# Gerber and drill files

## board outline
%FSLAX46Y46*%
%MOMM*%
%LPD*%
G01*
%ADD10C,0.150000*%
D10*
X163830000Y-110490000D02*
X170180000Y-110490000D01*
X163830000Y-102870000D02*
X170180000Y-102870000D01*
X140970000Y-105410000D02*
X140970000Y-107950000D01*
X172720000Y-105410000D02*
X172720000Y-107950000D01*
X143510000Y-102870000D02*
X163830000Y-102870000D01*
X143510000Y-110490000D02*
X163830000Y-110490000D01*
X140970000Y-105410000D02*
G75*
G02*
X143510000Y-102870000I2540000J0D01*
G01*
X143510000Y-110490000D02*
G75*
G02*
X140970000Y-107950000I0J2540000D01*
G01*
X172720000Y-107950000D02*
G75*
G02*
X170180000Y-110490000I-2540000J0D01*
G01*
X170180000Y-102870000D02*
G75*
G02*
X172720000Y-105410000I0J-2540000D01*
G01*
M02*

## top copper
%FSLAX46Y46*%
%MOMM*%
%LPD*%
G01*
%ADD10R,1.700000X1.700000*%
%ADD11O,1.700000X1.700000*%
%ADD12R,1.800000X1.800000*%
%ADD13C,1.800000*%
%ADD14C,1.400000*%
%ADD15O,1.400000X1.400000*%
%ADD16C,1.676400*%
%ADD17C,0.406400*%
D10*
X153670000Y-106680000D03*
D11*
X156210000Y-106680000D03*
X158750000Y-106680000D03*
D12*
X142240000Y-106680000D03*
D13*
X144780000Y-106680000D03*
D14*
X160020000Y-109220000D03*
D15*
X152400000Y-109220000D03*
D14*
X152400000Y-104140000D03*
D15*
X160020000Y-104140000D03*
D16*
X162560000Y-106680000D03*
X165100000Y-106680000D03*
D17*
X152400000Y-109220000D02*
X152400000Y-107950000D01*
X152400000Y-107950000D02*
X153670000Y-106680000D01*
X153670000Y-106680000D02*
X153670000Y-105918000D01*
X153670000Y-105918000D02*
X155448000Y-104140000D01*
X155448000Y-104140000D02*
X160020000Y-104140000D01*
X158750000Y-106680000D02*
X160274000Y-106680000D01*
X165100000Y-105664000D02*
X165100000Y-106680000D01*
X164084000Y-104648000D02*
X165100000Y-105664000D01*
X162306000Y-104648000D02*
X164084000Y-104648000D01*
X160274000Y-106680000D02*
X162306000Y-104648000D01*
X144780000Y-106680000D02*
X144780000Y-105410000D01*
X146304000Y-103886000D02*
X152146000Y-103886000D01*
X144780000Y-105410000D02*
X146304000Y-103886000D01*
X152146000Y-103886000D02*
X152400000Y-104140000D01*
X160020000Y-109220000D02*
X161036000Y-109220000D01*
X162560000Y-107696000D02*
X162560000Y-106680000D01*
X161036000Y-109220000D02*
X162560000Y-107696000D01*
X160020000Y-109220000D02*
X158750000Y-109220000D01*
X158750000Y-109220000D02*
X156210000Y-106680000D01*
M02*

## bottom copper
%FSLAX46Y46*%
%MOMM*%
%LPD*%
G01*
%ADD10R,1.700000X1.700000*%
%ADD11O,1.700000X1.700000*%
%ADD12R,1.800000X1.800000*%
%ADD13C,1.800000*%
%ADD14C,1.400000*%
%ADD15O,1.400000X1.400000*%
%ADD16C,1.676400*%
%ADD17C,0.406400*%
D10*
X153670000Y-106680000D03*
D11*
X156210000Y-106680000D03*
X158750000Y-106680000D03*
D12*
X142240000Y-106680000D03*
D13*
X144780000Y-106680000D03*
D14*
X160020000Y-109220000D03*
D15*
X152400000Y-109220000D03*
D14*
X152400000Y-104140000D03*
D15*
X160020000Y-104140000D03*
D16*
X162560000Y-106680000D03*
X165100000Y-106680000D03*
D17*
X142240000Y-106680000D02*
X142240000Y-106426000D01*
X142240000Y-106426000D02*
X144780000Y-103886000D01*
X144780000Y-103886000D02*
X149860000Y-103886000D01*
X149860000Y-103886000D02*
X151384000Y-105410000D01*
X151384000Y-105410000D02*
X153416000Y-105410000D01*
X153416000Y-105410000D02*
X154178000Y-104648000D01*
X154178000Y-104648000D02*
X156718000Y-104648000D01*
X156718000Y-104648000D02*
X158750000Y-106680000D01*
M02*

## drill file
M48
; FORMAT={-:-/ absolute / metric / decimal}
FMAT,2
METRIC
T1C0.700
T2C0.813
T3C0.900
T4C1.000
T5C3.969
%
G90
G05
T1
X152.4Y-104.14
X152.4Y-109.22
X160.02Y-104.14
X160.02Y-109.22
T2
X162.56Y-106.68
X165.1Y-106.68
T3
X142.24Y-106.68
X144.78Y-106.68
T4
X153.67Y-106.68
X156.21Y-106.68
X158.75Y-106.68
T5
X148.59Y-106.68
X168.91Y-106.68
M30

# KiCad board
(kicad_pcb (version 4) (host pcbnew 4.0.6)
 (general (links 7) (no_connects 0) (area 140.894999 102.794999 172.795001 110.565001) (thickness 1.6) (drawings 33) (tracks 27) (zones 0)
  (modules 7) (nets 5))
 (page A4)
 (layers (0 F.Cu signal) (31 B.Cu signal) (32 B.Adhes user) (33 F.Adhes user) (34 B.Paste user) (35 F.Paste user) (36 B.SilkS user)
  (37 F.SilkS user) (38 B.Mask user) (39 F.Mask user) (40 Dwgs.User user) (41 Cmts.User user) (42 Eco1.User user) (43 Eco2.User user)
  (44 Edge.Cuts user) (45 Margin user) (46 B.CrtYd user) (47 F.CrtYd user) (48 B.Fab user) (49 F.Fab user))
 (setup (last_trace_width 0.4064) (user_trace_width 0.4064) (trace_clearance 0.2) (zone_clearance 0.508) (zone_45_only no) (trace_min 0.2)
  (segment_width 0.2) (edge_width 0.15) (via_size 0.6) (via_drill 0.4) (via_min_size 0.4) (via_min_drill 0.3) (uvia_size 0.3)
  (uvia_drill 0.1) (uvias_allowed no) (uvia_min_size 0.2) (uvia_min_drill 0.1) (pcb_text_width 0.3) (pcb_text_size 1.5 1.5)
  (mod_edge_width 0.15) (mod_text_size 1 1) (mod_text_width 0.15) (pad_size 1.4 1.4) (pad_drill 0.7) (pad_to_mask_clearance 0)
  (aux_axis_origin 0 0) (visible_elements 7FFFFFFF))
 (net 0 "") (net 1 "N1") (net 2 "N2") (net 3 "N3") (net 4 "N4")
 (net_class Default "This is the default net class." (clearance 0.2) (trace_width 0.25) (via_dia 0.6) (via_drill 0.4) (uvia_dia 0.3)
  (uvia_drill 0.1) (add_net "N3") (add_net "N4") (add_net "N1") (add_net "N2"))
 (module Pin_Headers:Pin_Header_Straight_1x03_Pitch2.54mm (layer F.Cu) (at 153.67 106.68 90)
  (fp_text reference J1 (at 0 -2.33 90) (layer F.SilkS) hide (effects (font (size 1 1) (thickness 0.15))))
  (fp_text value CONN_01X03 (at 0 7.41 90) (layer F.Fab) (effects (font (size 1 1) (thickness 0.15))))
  (pad 1 thru_hole rect (at 0 0 90) (size 1.7 1.7) (drill 1) (layers *.Cu *.Mask) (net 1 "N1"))
  (pad 2 thru_hole oval (at 0 2.54 90) (size 1.7 1.7) (drill 1) (layers *.Cu *.Mask) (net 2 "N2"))
  (pad 3 thru_hole oval (at 0 5.08 90) (size 1.7 1.7) (drill 1) (layers *.Cu *.Mask) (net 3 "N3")))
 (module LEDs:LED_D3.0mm (layer F.Cu) (at 142.24 106.68)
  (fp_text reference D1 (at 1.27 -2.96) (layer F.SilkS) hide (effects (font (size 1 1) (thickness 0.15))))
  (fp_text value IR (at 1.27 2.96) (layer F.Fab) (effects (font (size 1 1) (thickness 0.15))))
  (pad 1 thru_hole rect (at 0 0) (size 1.8 1.8) (drill 0.9) (layers *.Cu B.Mask) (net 3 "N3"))
  (pad 2 thru_hole circle (at 2.54 0) (size 1.8 1.8) (drill 0.9) (layers *.Cu B.Mask) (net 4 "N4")))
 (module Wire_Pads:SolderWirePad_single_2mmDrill (layer F.Cu) (at 168.91 106.68)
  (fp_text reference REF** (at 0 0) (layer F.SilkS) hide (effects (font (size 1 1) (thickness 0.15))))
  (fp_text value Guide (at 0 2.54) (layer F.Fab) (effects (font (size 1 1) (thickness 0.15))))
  (pad "" np_thru_hole circle (at 0 0) (size 3.96875 3.96875) (drill 3.96875) (layers *.Cu *.Mask)))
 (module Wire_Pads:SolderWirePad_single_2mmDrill (layer F.Cu) (at 148.59 106.68)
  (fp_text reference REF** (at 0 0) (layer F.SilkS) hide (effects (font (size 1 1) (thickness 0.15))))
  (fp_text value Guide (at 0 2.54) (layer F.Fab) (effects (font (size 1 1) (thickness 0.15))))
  (pad "" np_thru_hole circle (at 0 0) (size 3.96875 3.96875) (drill 3.96875) (layers *.Cu *.Mask)))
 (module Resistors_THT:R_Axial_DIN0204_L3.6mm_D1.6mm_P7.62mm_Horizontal (layer F.Cu) (at 160.02 109.22 180)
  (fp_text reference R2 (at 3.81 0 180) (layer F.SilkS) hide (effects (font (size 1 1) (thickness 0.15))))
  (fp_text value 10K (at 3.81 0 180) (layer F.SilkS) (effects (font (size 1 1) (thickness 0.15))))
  (pad 1 thru_hole circle (at 0 0 180) (size 1.4 1.4) (drill 0.7) (layers *.Cu *.Mask) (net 2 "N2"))
  (pad 2 thru_hole oval (at 7.62 0 180) (size 1.4 1.4) (drill 0.7) (layers *.Cu *.Mask) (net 1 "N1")))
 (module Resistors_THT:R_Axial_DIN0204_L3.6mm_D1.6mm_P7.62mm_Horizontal (layer F.Cu) (at 152.4 104.14)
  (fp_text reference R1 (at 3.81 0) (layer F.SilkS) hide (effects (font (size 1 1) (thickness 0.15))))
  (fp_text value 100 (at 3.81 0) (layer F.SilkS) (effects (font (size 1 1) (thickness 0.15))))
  (pad 1 thru_hole circle (at 0 0) (size 1.4 1.4) (drill 0.7) (layers *.Cu *.Mask) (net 4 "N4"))
  (pad 2 thru_hole oval (at 7.62 0) (size 1.4 1.4) (drill 0.7) (layers *.Cu *.Mask) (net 1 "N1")))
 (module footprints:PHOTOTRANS (layer F.Cu) (at 163.83 106.68)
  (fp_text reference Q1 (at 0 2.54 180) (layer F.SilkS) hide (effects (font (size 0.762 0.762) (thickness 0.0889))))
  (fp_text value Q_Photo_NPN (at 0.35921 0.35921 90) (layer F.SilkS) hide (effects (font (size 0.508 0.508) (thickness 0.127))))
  (pad 1 thru_hole circle (at -1.27 0) (size 1.6764 1.6764) (drill 0.8128) (layers *.Cu B.Mask) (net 2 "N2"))
  (pad 2 thru_hole circle (at 1.27 0 45) (size 1.6764 1.6764) (drill 0.8128) (layers *.Cu B.Mask) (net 3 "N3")))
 (gr_line (start 163.83 110.49) (end 170.18 110.49) (angle 90) (layer Edge.Cuts) (width 0.15))
 (gr_line (start 163.83 102.87) (end 170.18 102.87) (angle 90) (layer Edge.Cuts) (width 0.15))
 (gr_line (start 140.97 105.41) (end 140.97 107.95) (angle 90) (layer Edge.Cuts) (width 0.15))
 (gr_line (start 172.72 105.41) (end 172.72 107.95) (angle 90) (layer Edge.Cuts) (width 0.15))
 (gr_line (start 143.51 102.87) (end 163.83 102.87) (angle 90) (layer Edge.Cuts) (width 0.15))
 (gr_line (start 143.51 110.49) (end 163.83 110.49) (angle 90) (layer Edge.Cuts) (width 0.15))
 (gr_arc (start 143.51 105.41) (end 140.97 105.41) (angle 90) (layer Edge.Cuts) (width 0.15))
 (gr_arc (start 143.51 107.95) (end 143.51 110.49) (angle 90) (layer Edge.Cuts) (width 0.15))
 (gr_arc (start 170.18 107.95) (end 172.72 107.95) (angle 90) (layer Edge.Cuts) (width 0.15))
 (gr_arc (start 170.18 105.41) (end 170.18 102.87) (angle 90) (layer Edge.Cuts) (width 0.15))
 (segment (start 152.4 109.22) (end 152.4 107.95) (width 0.4064) (layer F.Cu) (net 1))
 (segment (start 152.4 107.95) (end 153.67 106.68) (width 0.4064) (layer F.Cu) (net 1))
 (segment (start 153.67 106.68) (end 153.67 105.918) (width 0.4064) (layer F.Cu) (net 1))
 (segment (start 153.67 105.918) (end 155.448 104.14) (width 0.4064) (layer F.Cu) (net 1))
 (segment (start 155.448 104.14) (end 160.02 104.14) (width 0.4064) (layer F.Cu) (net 1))
 (segment (start 142.24 106.68) (end 142.24 106.426) (width 0.4064) (layer B.Cu) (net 3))
 (segment (start 142.24 106.426) (end 144.78 103.886) (width 0.4064) (layer B.Cu) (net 3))
 (segment (start 144.78 103.886) (end 149.86 103.886) (width 0.4064) (layer B.Cu) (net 3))
 (segment (start 149.86 103.886) (end 151.384 105.41) (width 0.4064) (layer B.Cu) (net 3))
 (segment (start 151.384 105.41) (end 153.416 105.41) (width 0.4064) (layer B.Cu) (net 3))
 (segment (start 153.416 105.41) (end 154.178 104.648) (width 0.4064) (layer B.Cu) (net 3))
 (segment (start 154.178 104.648) (end 156.718 104.648) (width 0.4064) (layer B.Cu) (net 3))
 (segment (start 156.718 104.648) (end 158.75 106.68) (width 0.4064) (layer B.Cu) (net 3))
 (segment (start 158.75 106.68) (end 160.274 106.68) (width 0.4064) (layer F.Cu) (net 3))
 (segment (start 165.1 105.664) (end 165.1 106.68) (width 0.4064) (layer F.Cu) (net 3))
 (segment (start 164.084 104.648) (end 165.1 105.664) (width 0.4064) (layer F.Cu) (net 3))
 (segment (start 162.306 104.648) (end 164.084 104.648) (width 0.4064) (layer F.Cu) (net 3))
 (segment (start 160.274 106.68) (end 162.306 104.648) (width 0.4064) (layer F.Cu) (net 3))
 (segment (start 144.78 106.68) (end 144.78 105.41) (width 0.4064) (layer F.Cu) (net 4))
 (segment (start 146.304 103.886) (end 152.146 103.886) (width 0.4064) (layer F.Cu) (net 4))
 (segment (start 144.78 105.41) (end 146.304 103.886) (width 0.4064) (layer F.Cu) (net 4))
 (segment (start 152.146 103.886) (end 152.4 104.14) (width 0.4064) (layer F.Cu) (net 4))
 (segment (start 160.02 109.22) (end 161.036 109.22) (width 0.4064) (layer F.Cu) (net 2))
 (segment (start 162.56 107.696) (end 162.56 106.68) (width 0.4064) (layer F.Cu) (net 2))
 (segment (start 161.036 109.22) (end 162.56 107.696) (width 0.4064) (layer F.Cu) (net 2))
 (segment (start 160.02 109.22) (end 158.75 109.22) (width 0.4064) (layer F.Cu) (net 2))
 (segment (start 158.75 109.22) (end 156.21 106.68) (width 0.4064) (layer F.Cu) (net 2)))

